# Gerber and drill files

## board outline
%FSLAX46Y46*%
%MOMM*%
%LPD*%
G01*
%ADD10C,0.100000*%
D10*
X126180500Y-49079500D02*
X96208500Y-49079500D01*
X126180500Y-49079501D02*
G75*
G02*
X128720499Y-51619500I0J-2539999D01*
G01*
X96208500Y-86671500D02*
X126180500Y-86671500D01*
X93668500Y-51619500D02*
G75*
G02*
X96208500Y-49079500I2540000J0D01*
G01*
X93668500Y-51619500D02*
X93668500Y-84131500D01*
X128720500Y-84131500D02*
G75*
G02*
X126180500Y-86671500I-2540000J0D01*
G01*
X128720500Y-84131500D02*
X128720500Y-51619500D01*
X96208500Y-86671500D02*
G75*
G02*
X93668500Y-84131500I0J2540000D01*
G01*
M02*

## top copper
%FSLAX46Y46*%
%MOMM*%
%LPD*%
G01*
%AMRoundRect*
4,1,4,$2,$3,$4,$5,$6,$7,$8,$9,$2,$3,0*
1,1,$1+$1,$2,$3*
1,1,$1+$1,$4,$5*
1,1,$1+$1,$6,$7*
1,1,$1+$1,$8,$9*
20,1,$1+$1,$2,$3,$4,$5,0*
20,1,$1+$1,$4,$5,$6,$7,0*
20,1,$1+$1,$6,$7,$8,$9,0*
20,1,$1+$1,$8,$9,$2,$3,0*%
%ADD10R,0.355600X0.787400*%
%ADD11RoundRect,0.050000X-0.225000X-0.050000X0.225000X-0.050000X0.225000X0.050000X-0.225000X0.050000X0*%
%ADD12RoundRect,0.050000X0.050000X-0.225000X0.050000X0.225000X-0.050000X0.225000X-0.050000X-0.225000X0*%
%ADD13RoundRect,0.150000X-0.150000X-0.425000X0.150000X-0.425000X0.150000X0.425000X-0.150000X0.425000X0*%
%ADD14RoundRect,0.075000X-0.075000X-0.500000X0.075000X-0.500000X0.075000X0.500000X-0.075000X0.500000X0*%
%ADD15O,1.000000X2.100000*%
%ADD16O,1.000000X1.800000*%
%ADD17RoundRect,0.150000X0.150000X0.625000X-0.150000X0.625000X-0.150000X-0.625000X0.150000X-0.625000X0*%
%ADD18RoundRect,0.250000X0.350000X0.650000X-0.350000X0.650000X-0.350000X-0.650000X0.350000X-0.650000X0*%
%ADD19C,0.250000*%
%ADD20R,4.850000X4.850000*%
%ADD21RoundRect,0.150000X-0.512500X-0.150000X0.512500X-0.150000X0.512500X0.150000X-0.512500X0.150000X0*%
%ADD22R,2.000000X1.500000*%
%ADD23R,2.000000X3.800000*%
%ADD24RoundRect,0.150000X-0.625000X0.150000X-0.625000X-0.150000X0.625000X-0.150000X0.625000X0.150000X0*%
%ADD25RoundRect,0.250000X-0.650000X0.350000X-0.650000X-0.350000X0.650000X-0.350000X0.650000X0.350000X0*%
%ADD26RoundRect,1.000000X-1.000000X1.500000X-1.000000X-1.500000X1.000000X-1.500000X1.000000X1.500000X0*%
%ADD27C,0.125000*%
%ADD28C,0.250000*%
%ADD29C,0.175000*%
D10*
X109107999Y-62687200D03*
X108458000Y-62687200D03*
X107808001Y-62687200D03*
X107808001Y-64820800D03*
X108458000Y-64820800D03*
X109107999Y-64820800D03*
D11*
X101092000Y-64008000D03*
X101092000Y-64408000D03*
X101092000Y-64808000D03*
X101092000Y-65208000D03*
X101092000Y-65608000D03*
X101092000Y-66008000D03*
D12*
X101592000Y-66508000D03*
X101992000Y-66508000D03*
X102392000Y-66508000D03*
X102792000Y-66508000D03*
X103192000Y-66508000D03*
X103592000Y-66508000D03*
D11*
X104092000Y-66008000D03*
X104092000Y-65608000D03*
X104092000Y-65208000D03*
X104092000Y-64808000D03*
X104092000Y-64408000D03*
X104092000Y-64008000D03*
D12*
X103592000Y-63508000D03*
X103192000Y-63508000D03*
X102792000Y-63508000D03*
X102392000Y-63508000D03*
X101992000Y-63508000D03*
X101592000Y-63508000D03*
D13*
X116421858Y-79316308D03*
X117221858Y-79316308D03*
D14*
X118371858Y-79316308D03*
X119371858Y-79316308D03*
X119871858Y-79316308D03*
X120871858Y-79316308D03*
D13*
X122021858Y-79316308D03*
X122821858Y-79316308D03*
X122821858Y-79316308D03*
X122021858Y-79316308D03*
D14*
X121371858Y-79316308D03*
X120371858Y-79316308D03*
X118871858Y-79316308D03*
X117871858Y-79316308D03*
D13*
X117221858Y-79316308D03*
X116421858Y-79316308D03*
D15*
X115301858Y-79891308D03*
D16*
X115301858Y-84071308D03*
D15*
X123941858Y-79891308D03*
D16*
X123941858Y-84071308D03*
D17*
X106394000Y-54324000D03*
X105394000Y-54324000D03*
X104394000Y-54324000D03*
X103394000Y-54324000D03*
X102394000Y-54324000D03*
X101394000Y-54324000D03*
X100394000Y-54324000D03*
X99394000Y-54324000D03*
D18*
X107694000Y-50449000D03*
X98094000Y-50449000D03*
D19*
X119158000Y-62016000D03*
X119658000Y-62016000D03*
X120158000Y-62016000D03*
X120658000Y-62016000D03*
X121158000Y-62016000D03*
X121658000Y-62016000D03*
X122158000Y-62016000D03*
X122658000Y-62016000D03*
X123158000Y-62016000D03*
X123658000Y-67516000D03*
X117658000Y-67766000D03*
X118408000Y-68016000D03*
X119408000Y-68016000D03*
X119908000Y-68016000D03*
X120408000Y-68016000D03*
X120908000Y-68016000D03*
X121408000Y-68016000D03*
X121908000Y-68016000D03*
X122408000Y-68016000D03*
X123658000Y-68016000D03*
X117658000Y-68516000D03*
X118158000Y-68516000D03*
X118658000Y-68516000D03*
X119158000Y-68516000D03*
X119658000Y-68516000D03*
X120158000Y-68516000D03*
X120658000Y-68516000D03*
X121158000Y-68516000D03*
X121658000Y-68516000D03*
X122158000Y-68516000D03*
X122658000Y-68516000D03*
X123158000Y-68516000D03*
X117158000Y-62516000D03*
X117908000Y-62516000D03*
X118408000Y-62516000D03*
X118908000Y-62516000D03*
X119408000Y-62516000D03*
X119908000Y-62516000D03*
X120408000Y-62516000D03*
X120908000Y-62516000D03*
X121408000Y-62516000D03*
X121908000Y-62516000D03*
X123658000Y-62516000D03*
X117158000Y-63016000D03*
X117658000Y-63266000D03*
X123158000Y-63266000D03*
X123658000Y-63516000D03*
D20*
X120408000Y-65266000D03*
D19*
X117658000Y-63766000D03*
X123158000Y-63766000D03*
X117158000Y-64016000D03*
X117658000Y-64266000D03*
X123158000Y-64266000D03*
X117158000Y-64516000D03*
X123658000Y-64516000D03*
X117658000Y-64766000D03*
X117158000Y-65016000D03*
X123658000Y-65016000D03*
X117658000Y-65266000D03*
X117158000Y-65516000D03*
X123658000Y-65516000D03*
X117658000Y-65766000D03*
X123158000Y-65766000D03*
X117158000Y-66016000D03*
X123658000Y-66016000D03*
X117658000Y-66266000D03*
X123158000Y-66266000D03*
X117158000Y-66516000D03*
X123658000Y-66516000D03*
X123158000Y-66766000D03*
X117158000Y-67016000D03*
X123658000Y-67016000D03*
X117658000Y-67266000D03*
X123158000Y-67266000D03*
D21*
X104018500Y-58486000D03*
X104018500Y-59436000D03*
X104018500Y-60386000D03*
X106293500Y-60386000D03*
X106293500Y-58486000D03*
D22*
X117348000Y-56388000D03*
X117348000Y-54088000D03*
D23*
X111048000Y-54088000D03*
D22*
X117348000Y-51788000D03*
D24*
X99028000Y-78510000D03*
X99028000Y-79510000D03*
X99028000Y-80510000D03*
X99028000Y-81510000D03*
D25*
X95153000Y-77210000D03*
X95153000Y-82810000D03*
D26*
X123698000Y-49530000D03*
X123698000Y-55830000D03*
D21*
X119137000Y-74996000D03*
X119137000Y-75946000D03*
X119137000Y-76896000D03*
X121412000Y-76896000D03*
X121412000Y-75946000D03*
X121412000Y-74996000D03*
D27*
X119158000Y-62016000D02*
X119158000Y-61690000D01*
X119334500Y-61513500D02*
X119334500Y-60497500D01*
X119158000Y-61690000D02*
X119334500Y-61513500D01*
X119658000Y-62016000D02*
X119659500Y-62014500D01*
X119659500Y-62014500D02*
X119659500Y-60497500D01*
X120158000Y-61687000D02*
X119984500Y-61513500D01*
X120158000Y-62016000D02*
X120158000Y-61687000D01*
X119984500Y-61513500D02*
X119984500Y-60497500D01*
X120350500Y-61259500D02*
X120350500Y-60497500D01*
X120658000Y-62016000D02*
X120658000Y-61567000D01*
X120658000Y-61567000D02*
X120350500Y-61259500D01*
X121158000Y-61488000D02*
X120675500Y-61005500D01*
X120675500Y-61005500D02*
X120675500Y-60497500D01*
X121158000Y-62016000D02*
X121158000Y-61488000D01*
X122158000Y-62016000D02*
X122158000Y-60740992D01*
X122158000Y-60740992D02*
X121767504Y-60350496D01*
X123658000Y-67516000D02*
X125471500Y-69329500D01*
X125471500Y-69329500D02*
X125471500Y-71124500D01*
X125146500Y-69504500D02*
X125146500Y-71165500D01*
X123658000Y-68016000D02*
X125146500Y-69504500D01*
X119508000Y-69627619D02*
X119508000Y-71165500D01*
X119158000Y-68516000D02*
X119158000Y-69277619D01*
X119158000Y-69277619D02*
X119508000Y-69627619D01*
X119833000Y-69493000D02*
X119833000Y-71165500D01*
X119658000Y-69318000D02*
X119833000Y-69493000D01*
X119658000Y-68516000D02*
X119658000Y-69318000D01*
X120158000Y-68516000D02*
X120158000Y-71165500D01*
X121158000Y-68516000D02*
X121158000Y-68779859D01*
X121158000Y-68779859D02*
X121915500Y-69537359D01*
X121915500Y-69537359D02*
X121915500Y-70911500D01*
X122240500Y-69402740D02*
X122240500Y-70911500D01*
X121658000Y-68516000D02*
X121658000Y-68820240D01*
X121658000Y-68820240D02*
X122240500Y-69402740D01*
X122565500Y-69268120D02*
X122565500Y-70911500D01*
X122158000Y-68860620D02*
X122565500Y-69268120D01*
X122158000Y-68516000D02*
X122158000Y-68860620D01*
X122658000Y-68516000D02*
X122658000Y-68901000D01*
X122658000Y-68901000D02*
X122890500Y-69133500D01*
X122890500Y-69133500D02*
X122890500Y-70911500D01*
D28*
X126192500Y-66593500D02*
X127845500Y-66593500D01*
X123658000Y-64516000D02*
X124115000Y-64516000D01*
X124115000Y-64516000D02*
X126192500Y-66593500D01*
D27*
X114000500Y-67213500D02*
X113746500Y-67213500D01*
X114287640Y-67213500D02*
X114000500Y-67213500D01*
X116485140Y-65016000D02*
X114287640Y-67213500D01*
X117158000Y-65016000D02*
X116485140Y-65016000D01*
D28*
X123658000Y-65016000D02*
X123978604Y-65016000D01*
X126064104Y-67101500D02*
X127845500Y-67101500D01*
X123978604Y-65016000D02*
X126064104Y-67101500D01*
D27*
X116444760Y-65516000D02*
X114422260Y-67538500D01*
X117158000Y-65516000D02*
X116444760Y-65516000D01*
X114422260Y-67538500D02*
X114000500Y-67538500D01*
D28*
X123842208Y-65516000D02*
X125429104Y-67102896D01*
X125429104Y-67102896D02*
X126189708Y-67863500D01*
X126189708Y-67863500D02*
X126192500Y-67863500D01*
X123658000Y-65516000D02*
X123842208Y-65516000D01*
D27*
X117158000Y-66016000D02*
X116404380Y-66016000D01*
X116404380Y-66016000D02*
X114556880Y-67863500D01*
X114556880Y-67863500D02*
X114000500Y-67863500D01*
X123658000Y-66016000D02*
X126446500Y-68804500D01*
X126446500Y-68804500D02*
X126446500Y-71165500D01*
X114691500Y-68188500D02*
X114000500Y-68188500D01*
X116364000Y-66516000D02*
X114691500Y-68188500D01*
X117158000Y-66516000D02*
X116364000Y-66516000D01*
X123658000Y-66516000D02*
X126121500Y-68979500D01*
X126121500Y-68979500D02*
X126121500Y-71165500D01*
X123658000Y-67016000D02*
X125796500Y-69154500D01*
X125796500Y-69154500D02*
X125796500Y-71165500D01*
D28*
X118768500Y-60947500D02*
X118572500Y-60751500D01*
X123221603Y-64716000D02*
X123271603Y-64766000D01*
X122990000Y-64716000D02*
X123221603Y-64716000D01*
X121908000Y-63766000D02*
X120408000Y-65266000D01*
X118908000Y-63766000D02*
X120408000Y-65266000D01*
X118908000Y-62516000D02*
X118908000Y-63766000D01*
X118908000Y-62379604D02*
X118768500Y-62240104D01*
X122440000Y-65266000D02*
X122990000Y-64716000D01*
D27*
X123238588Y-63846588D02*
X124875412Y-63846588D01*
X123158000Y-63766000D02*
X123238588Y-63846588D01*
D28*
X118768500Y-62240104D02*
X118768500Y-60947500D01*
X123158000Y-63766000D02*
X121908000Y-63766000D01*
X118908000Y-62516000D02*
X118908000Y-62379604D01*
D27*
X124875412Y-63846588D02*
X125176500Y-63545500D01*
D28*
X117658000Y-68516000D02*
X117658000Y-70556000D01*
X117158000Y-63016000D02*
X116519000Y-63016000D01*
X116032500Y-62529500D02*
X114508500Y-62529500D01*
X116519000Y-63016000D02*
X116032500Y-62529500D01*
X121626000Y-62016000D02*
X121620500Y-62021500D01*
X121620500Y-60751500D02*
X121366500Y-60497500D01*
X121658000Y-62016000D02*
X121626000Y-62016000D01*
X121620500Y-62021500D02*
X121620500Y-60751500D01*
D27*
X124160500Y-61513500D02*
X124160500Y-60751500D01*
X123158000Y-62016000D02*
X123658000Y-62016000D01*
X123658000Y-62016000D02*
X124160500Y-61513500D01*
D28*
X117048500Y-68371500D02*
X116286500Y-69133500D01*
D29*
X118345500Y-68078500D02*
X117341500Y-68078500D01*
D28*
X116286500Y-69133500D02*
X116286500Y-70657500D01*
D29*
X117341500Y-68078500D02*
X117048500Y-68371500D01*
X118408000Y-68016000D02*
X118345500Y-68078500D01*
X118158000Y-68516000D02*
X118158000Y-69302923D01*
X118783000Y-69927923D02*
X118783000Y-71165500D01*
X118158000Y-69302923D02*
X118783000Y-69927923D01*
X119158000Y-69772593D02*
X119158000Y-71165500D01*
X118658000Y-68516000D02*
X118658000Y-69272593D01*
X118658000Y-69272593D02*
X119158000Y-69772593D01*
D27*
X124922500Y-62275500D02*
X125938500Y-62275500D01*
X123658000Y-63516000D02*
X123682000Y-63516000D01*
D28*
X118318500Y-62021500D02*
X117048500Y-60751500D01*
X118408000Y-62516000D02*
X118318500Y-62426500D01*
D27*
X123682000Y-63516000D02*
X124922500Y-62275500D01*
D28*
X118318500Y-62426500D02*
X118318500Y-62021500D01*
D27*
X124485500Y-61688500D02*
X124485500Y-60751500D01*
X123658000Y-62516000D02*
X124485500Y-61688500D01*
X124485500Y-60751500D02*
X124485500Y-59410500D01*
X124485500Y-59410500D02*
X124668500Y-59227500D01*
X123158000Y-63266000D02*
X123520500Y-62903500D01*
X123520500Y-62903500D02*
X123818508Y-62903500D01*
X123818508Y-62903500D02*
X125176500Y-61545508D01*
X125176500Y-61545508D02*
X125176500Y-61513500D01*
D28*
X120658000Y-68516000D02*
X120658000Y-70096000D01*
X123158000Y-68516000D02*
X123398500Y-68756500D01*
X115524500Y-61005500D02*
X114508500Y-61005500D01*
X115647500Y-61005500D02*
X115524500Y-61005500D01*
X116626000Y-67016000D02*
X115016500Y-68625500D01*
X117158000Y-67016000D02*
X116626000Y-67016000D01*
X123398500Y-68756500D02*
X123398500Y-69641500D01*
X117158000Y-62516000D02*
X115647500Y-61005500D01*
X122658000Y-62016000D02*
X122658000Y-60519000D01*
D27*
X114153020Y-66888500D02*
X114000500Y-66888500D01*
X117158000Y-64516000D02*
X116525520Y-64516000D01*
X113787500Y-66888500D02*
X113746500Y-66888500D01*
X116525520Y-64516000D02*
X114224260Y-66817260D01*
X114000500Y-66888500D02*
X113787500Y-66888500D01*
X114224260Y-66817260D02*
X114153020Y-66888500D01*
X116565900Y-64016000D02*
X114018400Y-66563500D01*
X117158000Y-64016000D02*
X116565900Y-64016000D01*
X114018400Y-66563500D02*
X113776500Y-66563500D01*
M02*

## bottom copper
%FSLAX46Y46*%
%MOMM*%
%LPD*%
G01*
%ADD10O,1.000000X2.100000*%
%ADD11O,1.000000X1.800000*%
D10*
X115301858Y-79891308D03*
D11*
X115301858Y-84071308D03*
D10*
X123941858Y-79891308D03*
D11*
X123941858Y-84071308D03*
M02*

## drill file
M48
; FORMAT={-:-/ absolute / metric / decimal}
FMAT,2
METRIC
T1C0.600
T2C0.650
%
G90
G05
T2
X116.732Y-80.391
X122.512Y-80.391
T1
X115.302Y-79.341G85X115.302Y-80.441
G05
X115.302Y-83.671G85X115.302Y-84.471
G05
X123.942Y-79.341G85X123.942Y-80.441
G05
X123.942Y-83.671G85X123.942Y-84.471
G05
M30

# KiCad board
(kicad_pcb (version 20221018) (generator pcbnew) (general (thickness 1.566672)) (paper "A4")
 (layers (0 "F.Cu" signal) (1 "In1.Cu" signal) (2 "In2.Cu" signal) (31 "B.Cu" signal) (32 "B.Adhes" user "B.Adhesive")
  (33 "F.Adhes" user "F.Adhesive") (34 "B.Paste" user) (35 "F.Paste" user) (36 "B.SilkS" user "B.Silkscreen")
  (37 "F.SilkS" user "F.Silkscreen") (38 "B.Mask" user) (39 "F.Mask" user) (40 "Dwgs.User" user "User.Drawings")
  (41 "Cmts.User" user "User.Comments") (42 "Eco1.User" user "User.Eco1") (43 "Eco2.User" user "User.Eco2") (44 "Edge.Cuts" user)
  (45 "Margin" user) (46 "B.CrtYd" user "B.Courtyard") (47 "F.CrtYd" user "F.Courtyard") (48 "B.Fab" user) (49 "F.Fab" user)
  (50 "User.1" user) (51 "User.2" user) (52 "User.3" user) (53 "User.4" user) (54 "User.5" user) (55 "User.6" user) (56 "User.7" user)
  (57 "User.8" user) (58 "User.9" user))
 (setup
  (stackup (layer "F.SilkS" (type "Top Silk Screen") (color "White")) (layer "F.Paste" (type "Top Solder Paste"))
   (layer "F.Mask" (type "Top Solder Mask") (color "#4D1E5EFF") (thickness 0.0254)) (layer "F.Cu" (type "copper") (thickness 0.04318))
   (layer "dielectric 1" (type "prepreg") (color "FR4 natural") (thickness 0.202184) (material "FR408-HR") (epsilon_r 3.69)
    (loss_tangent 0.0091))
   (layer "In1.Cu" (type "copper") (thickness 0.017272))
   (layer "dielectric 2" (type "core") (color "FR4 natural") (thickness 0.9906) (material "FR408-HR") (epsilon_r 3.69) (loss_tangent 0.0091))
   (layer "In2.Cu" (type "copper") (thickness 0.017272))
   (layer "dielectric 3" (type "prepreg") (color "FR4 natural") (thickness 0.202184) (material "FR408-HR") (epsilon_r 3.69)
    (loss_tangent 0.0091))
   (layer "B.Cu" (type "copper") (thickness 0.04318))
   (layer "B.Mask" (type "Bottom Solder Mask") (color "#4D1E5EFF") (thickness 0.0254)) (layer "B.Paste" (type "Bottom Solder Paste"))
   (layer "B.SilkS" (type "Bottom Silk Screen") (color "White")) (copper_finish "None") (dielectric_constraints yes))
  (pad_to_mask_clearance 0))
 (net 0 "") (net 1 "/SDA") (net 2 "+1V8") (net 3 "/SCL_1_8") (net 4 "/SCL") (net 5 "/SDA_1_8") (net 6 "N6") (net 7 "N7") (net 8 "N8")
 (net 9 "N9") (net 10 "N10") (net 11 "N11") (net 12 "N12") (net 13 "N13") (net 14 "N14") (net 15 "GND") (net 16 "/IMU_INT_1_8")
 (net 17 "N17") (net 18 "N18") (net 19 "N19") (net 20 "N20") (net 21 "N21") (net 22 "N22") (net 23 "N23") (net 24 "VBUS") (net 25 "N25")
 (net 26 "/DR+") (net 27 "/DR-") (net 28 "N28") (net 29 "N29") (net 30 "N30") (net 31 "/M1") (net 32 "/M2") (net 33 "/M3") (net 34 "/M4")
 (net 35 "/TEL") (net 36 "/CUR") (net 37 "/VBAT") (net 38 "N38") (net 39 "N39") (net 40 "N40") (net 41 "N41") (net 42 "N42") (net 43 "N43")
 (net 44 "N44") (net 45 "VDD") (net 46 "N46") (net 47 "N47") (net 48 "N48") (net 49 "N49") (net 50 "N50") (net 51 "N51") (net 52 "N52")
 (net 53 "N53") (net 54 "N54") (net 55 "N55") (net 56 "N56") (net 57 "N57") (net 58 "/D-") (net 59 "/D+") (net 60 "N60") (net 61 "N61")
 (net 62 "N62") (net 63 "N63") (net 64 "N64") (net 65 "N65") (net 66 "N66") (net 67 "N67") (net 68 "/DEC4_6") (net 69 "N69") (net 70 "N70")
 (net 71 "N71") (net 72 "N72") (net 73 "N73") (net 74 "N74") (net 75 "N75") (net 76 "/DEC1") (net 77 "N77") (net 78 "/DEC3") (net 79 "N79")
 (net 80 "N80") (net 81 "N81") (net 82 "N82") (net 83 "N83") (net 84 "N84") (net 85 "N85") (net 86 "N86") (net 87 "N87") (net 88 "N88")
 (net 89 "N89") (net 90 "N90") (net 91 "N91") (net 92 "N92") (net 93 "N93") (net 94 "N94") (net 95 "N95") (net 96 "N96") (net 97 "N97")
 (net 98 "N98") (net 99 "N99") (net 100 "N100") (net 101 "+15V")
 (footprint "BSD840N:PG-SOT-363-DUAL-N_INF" (layer "F.Cu") (at 108.458 63.754 -90)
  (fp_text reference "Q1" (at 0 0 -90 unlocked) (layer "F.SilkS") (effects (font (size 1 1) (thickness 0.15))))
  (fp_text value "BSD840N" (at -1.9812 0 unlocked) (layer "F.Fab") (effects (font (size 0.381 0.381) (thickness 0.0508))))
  (pad "1" smd rect (at -1.0668 -0.649999 270) (size 0.7874 0.3556) (layers "F.Cu" "F.Paste" "F.Mask") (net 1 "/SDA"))
  (pad "2" smd rect (at -1.0668 0 270) (size 0.7874 0.3556) (layers "F.Cu" "F.Paste" "F.Mask") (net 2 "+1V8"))
  (pad "3" smd rect (at -1.0668 0.649999 270) (size 0.7874 0.3556) (layers "F.Cu" "F.Paste" "F.Mask") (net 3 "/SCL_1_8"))
  (pad "4" smd rect (at 1.0668 0.649999 270) (size 0.7874 0.3556) (layers "F.Cu" "F.Paste" "F.Mask") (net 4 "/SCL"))
  (pad "5" smd rect (at 1.0668 0 270) (size 0.7874 0.3556) (layers "F.Cu" "F.Paste" "F.Mask") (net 2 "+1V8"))
  (pad "6" smd rect (at 1.0668 -0.649999 270) (size 0.7874 0.3556) (layers "F.Cu" "F.Paste" "F.Mask") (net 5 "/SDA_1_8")))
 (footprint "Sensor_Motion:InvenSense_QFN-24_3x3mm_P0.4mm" (layer "F.Cu") (at 102.592 65.008)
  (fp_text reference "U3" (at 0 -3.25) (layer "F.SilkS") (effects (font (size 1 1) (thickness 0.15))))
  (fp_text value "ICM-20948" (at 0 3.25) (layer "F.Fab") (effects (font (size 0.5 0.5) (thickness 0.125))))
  (pad "1" smd roundrect (at -1.5 -1) (size 0.55 0.2) (layers "F.Cu" "F.Paste" "F.Mask") (roundrect_rratio 0.25) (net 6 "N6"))
  (pad "2" smd roundrect (at -1.5 -0.6) (size 0.55 0.2) (layers "F.Cu" "F.Paste" "F.Mask") (roundrect_rratio 0.25) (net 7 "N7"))
  (pad "3" smd roundrect (at -1.5 -0.2) (size 0.55 0.2) (layers "F.Cu" "F.Paste" "F.Mask") (roundrect_rratio 0.25) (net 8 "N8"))
  (pad "4" smd roundrect (at -1.5 0.2) (size 0.55 0.2) (layers "F.Cu" "F.Paste" "F.Mask") (roundrect_rratio 0.25) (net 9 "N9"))
  (pad "5" smd roundrect (at -1.5 0.6) (size 0.55 0.2) (layers "F.Cu" "F.Paste" "F.Mask") (roundrect_rratio 0.25) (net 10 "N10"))
  (pad "6" smd roundrect (at -1.5 1) (size 0.55 0.2) (layers "F.Cu" "F.Paste" "F.Mask") (roundrect_rratio 0.25) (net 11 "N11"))
  (pad "7" smd roundrect (at -1 1.5 90) (size 0.55 0.2) (layers "F.Cu" "F.Paste" "F.Mask") (roundrect_rratio 0.25) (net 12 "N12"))
  (pad "8" smd roundrect (at -0.6 1.5 90) (size 0.55 0.2) (layers "F.Cu" "F.Paste" "F.Mask") (roundrect_rratio 0.25) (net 2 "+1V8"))
  (pad "9" smd roundrect (at -0.2 1.5 90) (size 0.55 0.2) (layers "F.Cu" "F.Paste" "F.Mask") (roundrect_rratio 0.25) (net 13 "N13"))
  (pad "10" smd roundrect (at 0.2 1.5 90) (size 0.55 0.2) (layers "F.Cu" "F.Paste" "F.Mask") (roundrect_rratio 0.25) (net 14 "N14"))
  (pad "11" smd roundrect (at 0.6 1.5 90) (size 0.55 0.2) (layers "F.Cu" "F.Paste" "F.Mask") (roundrect_rratio 0.25) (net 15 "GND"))
  (pad "12" smd roundrect (at 1 1.5 90) (size 0.55 0.2) (layers "F.Cu" "F.Paste" "F.Mask") (roundrect_rratio 0.25) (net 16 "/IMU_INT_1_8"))
  (pad "13" smd roundrect (at 1.5 1) (size 0.55 0.2) (layers "F.Cu" "F.Paste" "F.Mask") (roundrect_rratio 0.25) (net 2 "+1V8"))
  (pad "14" smd roundrect (at 1.5 0.6) (size 0.55 0.2) (layers "F.Cu" "F.Paste" "F.Mask") (roundrect_rratio 0.25) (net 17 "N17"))
  (pad "15" smd roundrect (at 1.5 0.2) (size 0.55 0.2) (layers "F.Cu" "F.Paste" "F.Mask") (roundrect_rratio 0.25) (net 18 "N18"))
  (pad "16" smd roundrect (at 1.5 -0.2) (size 0.55 0.2) (layers "F.Cu" "F.Paste" "F.Mask") (roundrect_rratio 0.25) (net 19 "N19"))
  (pad "17" smd roundrect (at 1.5 -0.6) (size 0.55 0.2) (layers "F.Cu" "F.Paste" "F.Mask") (roundrect_rratio 0.25) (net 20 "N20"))
  (pad "18" smd roundrect (at 1.5 -1) (size 0.55 0.2) (layers "F.Cu" "F.Paste" "F.Mask") (roundrect_rratio 0.25) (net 15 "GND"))
  (pad "19" smd roundrect (at 1 -1.5 90) (size 0.55 0.2) (layers "F.Cu" "F.Paste" "F.Mask") (roundrect_rratio 0.25) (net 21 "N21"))
  (pad "20" smd roundrect (at 0.6 -1.5 90) (size 0.55 0.2) (layers "F.Cu" "F.Paste" "F.Mask") (roundrect_rratio 0.25) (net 15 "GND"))
  (pad "21" smd roundrect (at 0.2 -1.5 90) (size 0.55 0.2) (layers "F.Cu" "F.Paste" "F.Mask") (roundrect_rratio 0.25) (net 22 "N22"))
  (pad "22" smd roundrect (at -0.2 -1.5 90) (size 0.55 0.2) (layers "F.Cu" "F.Paste" "F.Mask") (roundrect_rratio 0.25) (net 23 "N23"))
  (pad "23" smd roundrect (at -0.6 -1.5 90) (size 0.55 0.2) (layers "F.Cu" "F.Paste" "F.Mask") (roundrect_rratio 0.25) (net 3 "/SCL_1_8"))
  (pad "24" smd roundrect (at -1 -1.5 90) (size 0.55 0.2) (layers "F.Cu" "F.Paste" "F.Mask") (roundrect_rratio 0.25) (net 5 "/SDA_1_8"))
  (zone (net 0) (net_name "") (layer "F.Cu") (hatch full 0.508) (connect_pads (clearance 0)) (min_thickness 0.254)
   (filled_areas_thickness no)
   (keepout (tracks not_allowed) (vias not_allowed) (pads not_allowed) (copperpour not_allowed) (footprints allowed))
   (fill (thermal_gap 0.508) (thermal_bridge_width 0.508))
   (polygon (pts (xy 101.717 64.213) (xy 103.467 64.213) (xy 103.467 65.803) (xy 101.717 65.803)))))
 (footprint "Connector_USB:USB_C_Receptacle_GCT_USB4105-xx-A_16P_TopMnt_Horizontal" (layer "F.Cu") (at 119.621858 82.996308)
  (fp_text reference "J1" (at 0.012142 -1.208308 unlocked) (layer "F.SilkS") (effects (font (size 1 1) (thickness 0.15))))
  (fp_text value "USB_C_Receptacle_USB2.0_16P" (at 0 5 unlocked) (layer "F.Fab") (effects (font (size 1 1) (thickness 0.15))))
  (pad "" np_thru_hole circle (at -2.89 -2.605) (size 0.65 0.65) (drill 0.65) (layers "F&B.Cu" "*.Mask"))
  (pad "" np_thru_hole circle (at 2.89 -2.605) (size 0.65 0.65) (drill 0.65) (layers "F&B.Cu" "*.Mask"))
  (pad "A1" smd roundrect (at -3.2 -3.68) (size 0.6 1.15) (layers "F.Cu" "F.Paste" "F.Mask") (roundrect_rratio 0.25) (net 15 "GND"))
  (pad "A4" smd roundrect (at -2.4 -3.68) (size 0.6 1.15) (layers "F.Cu" "F.Paste" "F.Mask") (roundrect_rratio 0.25) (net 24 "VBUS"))
  (pad "A5" smd roundrect (at -1.25 -3.68) (size 0.3 1.15) (layers "F.Cu" "F.Paste" "F.Mask") (roundrect_rratio 0.25) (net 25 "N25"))
  (pad "A6" smd roundrect (at -0.25 -3.68) (size 0.3 1.15) (layers "F.Cu" "F.Paste" "F.Mask") (roundrect_rratio 0.25) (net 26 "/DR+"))
  (pad "A7" smd roundrect (at 0.25 -3.68) (size 0.3 1.15) (layers "F.Cu" "F.Paste" "F.Mask") (roundrect_rratio 0.25) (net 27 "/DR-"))
  (pad "A8" smd roundrect (at 1.25 -3.68) (size 0.3 1.15) (layers "F.Cu" "F.Paste" "F.Mask") (roundrect_rratio 0.25) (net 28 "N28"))
  (pad "A9" smd roundrect (at 2.4 -3.68) (size 0.6 1.15) (layers "F.Cu" "F.Paste" "F.Mask") (roundrect_rratio 0.25) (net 24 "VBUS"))
  (pad "A12" smd roundrect (at 3.2 -3.68) (size 0.6 1.15) (layers "F.Cu" "F.Paste" "F.Mask") (roundrect_rratio 0.25) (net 15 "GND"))
  (pad "B1" smd roundrect (at 3.2 -3.68) (size 0.6 1.15) (layers "F.Cu" "F.Paste" "F.Mask") (roundrect_rratio 0.25) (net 15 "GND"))
  (pad "B4" smd roundrect (at 2.4 -3.68) (size 0.6 1.15) (layers "F.Cu" "F.Paste" "F.Mask") (roundrect_rratio 0.25) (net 24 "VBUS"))
  (pad "B5" smd roundrect (at 1.75 -3.68) (size 0.3 1.15) (layers "F.Cu" "F.Paste" "F.Mask") (roundrect_rratio 0.25) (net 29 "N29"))
  (pad "B6" smd roundrect (at 0.75 -3.68) (size 0.3 1.15) (layers "F.Cu" "F.Paste" "F.Mask") (roundrect_rratio 0.25) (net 26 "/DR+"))
  (pad "B7" smd roundrect (at -0.75 -3.68) (size 0.3 1.15) (layers "F.Cu" "F.Paste" "F.Mask") (roundrect_rratio 0.25) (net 27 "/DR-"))
  (pad "B8" smd roundrect (at -1.75 -3.68) (size 0.3 1.15) (layers "F.Cu" "F.Paste" "F.Mask") (roundrect_rratio 0.25) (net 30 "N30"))
  (pad "B9" smd roundrect (at -2.4 -3.68) (size 0.6 1.15) (layers "F.Cu" "F.Paste" "F.Mask") (roundrect_rratio 0.25) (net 24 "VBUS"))
  (pad "B12" smd roundrect (at -3.2 -3.68) (size 0.6 1.15) (layers "F.Cu" "F.Paste" "F.Mask") (roundrect_rratio 0.25) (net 15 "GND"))
  (pad "S1" thru_hole oval (at -4.32 -3.105) (size 1 2.1) (drill oval 0.6 1.7) (layers "*.Cu" "*.Mask" "F.Paste") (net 15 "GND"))
  (pad "S1" thru_hole oval (at -4.32 1.075) (size 1 1.8) (drill oval 0.6 1.4) (layers "*.Cu" "*.Mask" "F.Paste") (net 15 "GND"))
  (pad "S1" thru_hole oval (at 4.32 -3.105) (size 1 2.1) (drill oval 0.6 1.7) (layers "*.Cu" "*.Mask" "F.Paste") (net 15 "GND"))
  (pad "S1" thru_hole oval (at 4.32 1.075) (size 1 1.8) (drill oval 0.6 1.4) (layers "*.Cu" "*.Mask" "F.Paste") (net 15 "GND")))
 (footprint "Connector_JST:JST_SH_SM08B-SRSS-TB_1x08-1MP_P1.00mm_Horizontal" (layer "F.Cu") (at 102.894 52.324 180)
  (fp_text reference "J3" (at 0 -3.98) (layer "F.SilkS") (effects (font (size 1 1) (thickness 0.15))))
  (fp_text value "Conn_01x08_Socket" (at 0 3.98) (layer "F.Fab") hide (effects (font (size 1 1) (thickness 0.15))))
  (pad "1" smd roundrect (at -3.5 -2 180) (size 0.6 1.55) (layers "F.Cu" "F.Paste" "F.Mask") (roundrect_rratio 0.25) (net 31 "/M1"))
  (pad "2" smd roundrect (at -2.5 -2 180) (size 0.6 1.55) (layers "F.Cu" "F.Paste" "F.Mask") (roundrect_rratio 0.25) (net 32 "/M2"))
  (pad "3" smd roundrect (at -1.5 -2 180) (size 0.6 1.55) (layers "F.Cu" "F.Paste" "F.Mask") (roundrect_rratio 0.25) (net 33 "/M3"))
  (pad "4" smd roundrect (at -0.5 -2 180) (size 0.6 1.55) (layers "F.Cu" "F.Paste" "F.Mask") (roundrect_rratio 0.25) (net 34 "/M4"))
  (pad "5" smd roundrect (at 0.5 -2 180) (size 0.6 1.55) (layers "F.Cu" "F.Paste" "F.Mask") (roundrect_rratio 0.25) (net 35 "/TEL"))
  (pad "6" smd roundrect (at 1.5 -2 180) (size 0.6 1.55) (layers "F.Cu" "F.Paste" "F.Mask") (roundrect_rratio 0.25) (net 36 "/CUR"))
  (pad "7" smd roundrect (at 2.5 -2 180) (size 0.6 1.55) (layers "F.Cu" "F.Paste" "F.Mask") (roundrect_rratio 0.25) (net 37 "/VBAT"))
  (pad "8" smd roundrect (at 3.5 -2 180) (size 0.6 1.55) (layers "F.Cu" "F.Paste" "F.Mask") (roundrect_rratio 0.25) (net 15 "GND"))
  (pad "MP" smd roundrect (at -4.8 1.875 180) (size 1.2 1.8) (layers "F.Cu" "F.Paste" "F.Mask") (roundrect_rratio 0.208333))
  (pad "MP" smd roundrect (at 4.8 1.875 180) (size 1.2 1.8) (layers "F.Cu" "F.Paste" "F.Mask") (roundrect_rratio 0.208333)))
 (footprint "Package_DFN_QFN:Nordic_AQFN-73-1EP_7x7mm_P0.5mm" (layer "F.Cu") (at 120.408 65.266)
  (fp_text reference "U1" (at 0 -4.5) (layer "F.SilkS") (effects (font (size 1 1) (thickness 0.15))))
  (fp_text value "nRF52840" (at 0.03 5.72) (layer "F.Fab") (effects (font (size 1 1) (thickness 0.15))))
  (pad "" smd rect (at -1.2125 -1.2125 180) (size 2 2) (layers "F.Paste"))
  (pad "" smd rect (at -1.2125 1.2125 180) (size 2 2) (layers "F.Paste"))
  (pad "" smd rect (at 1.2125 -1.2125 180) (size 2 2) (layers "F.Paste"))
  (pad "" smd rect (at 1.2125 1.2125 180) (size 2 2) (layers "F.Paste"))
  (pad "A8" smd circle (at -1.25 -3.25 180) (size 0.25 0.25) (layers "F.Cu" "F.Paste" "F.Mask") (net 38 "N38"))
  (pad "A10" smd circle (at -0.75 -3.25 180) (size 0.25 0.25) (layers "F.Cu" "F.Paste" "F.Mask") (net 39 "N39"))
  (pad "A12" smd circle (at -0.25 -3.25 180) (size 0.25 0.25) (layers "F.Cu" "F.Paste" "F.Mask") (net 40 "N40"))
  (pad "A14" smd circle (at 0.25 -3.25 180) (size 0.25 0.25) (layers "F.Cu" "F.Paste" "F.Mask") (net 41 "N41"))
  (pad "A16" smd circle (at 0.75 -3.25 180) (size 0.25 0.25) (layers "F.Cu" "F.Paste" "F.Mask") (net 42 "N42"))
  (pad "A18" smd circle (at 1.25 -3.25 180) (size 0.25 0.25) (layers "F.Cu" "F.Paste" "F.Mask") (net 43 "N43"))
  (pad "A20" smd circle (at 1.75 -3.25 180) (size 0.25 0.25) (layers "F.Cu" "F.Paste" "F.Mask") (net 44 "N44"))
  (pad "A22" smd circle (at 2.25 -3.25 180) (size 0.25 0.25) (layers "F.Cu" "F.Paste" "F.Mask") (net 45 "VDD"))
  (pad "A23" smd circle (at 2.75 -3.25 180) (size 0.25 0.25) (layers "F.Cu" "F.Paste" "F.Mask") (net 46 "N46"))
  (pad "AA24" smd circle (at 3.25 2.25 180) (size 0.25 0.25) (layers "F.Cu" "F.Paste" "F.Mask") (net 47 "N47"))
  (pad "AB2" smd circle (at -2.75 2.5 180) (size 0.25 0.25) (layers "F.Cu" "F.Paste" "F.Mask") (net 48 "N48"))
  (pad "AC5" smd circle (at -2 2.75 180) (size 0.25 0.25) (layers "F.Cu" "F.Paste" "F.Mask") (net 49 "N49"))
  (pad "AC9" smd circle (at -1 2.75 180) (size 0.25 0.25) (layers "F.Cu" "F.Paste" "F.Mask") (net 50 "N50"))
  (pad "AC11" smd circle (at -0.5 2.75 180) (size 0.25 0.25) (layers "F.Cu" "F.Paste" "F.Mask") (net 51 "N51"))
  (pad "AC13" smd circle (at 0 2.75 180) (size 0.25 0.25) (layers "F.Cu" "F.Paste" "F.Mask") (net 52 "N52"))
  (pad "AC15" smd circle (at 0.5 2.75 180) (size 0.25 0.25) (layers "F.Cu" "F.Paste" "F.Mask") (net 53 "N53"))
  (pad "AC17" smd circle (at 1 2.75 180) (size 0.25 0.25) (layers "F.Cu" "F.Paste" "F.Mask") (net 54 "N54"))
  (pad "AC19" smd circle (at 1.5 2.75 180) (size 0.25 0.25) (layers "F.Cu" "F.Paste" "F.Mask") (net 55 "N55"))
  (pad "AC21" smd circle (at 2 2.75 180) (size 0.25 0.25) (layers "F.Cu" "F.Paste" "F.Mask") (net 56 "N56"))
  (pad "AC24" smd circle (at 3.25 2.75 180) (size 0.25 0.25) (layers "F.Cu" "F.Paste" "F.Mask") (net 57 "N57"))
  (pad "AD2" smd circle (at -2.75 3.25 180) (size 0.25 0.25) (layers "F.Cu" "F.Paste" "F.Mask") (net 24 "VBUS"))
  (pad "AD4" smd circle (at -2.25 3.25 180) (size 0.25 0.25) (layers "F.Cu" "F.Paste" "F.Mask") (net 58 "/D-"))
  (pad "AD6" smd circle (at -1.75 3.25 180) (size 0.25 0.25) (layers "F.Cu" "F.Paste" "F.Mask") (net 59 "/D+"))
  (pad "AD8" smd circle (at -1.25 3.25 180) (size 0.25 0.25) (layers "F.Cu" "F.Paste" "F.Mask") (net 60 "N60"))
  (pad "AD10" smd circle (at -0.75 3.25 180) (size 0.25 0.25) (layers "F.Cu" "F.Paste" "F.Mask") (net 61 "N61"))
  (pad "AD12" smd circle (at -0.25 3.25 180) (size 0.25 0.25) (layers "F.Cu" "F.Paste" "F.Mask") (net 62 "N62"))
  (pad "AD14" smd circle (at 0.25 3.25 180) (size 0.25 0.25) (layers "F.Cu" "F.Paste" "F.Mask") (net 45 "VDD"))
  (pad "AD16" smd circle (at 0.75 3.25 180) (size 0.25 0.25) (layers "F.Cu" "F.Paste" "F.Mask") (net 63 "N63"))
  (pad "AD18" smd circle (at 1.25 3.25 180) (size 0.25 0.25) (layers "F.Cu" "F.Paste" "F.Mask") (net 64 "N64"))
  (pad "AD20" smd circle (at 1.75 3.25 180) (size 0.25 0.25) (layers "F.Cu" "F.Paste" "F.Mask") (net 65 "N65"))
  (pad "AD22" smd circle (at 2.25 3.25 180) (size 0.25 0.25) (layers "F.Cu" "F.Paste" "F.Mask") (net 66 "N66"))
  (pad "AD23" smd circle (at 2.75 3.25 180) (size 0.25 0.25) (layers "F.Cu" "F.Paste" "F.Mask") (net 45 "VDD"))
  (pad "B1" smd circle (at -3.25 -2.75 180) (size 0.25 0.25) (layers "F.Cu" "F.Paste" "F.Mask") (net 45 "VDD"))
  (pad "B3" smd circle (at -2.5 -2.75 180) (size 0.25 0.25) (layers "F.Cu" "F.Paste" "F.Mask") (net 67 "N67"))
  (pad "B5" smd circle (at -2 -2.75 180) (size 0.25 0.25) (layers "F.Cu" "F.Paste" "F.Mask") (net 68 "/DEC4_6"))
  (pad "B7" smd circle (at -1.5 -2.75 180) (size 0.25 0.25) (layers "F.Cu" "F.Paste" "F.Mask") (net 15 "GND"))
  (pad "B9" smd circle (at -1 -2.75 180) (size 0.25 0.25) (layers "F.Cu" "F.Paste" "F.Mask") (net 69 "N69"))
  (pad "B11" smd circle (at -0.5 -2.75 180) (size 0.25 0.25) (layers "F.Cu" "F.Paste" "F.Mask") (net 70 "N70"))
  (pad "B13" smd circle (at 0 -2.75 180) (size 0.25 0.25) (layers "F.Cu" "F.Paste" "F.Mask") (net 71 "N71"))
  (pad "B15" smd circle (at 0.5 -2.75 180) (size 0.25 0.25) (layers "F.Cu" "F.Paste" "F.Mask") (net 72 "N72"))
  (pad "B17" smd circle (at 1 -2.75 180) (size 0.25 0.25) (layers "F.Cu" "F.Paste" "F.Mask") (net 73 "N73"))
  (pad "B19" smd circle (at 1.5 -2.75 180) (size 0.25 0.25) (layers "F.Cu" "F.Paste" "F.Mask") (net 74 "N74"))
  (pad "B24" smd circle (at 3.25 -2.75 180) (size 0.25 0.25) (layers "F.Cu" "F.Paste" "F.Mask") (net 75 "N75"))
  (pad "C1" smd circle (at -3.25 -2.25 180) (size 0.25 0.25) (layers "F.Cu" "F.Paste" "F.Mask") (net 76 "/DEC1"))
  (pad "D2" smd circle (at -2.75 -2 180) (size 0.25 0.25) (layers "F.Cu" "F.Paste" "F.Mask") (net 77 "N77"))
  (pad "D23" smd circle (at 2.75 -2 180) (size 0.25 0.25) (layers "F.Cu" "F.Paste" "F.Mask") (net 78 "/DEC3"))
  (pad "E24" smd circle (at 3.25 -1.75 180) (size 0.25 0.25) (layers "F.Cu" "F.Paste" "F.Mask") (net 68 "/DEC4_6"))
  (pad "EP" smd rect (at 0 0 180) (size 4.85 4.85) (layers "F.Cu" "F.Mask"))
  (pad "F2" smd circle (at -2.75 -1.5 180) (size 0.25 0.25) (layers "F.Cu" "F.Paste" "F.Mask") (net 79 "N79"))
  (pad "F23" smd circle (at 2.75 -1.5 180) (size 0.25 0.25) (layers "F.Cu" "F.Paste" "F.Mask") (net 15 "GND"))
  (pad "G1" smd circle (at -3.25 -1.25 180) (size 0.25 0.25) (layers "F.Cu" "F.Paste" "F.Mask") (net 1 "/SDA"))
  (pad "H2" smd circle (at -2.75 -1 180) (size 0.25 0.25) (layers "F.Cu" "F.Paste" "F.Mask") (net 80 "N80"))
  (pad "H23" smd circle (at 2.75 -1 180) (size 0.25 0.25) (layers "F.Cu" "F.Paste" "F.Mask") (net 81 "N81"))
  (pad "J1" smd circle (at -3.25 -0.75 180) (size 0.25 0.25) (layers "F.Cu" "F.Paste" "F.Mask") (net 4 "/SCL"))
  (pad "J24" smd circle (at 3.25 -0.75 180) (size 0.25 0.25) (layers "F.Cu" "F.Paste" "F.Mask") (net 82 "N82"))
  (pad "K2" smd circle (at -2.75 -0.5 180) (size 0.25 0.25) (layers "F.Cu" "F.Paste" "F.Mask") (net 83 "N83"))
  (pad "L1" smd circle (at -3.25 -0.25 180) (size 0.25 0.25) (layers "F.Cu" "F.Paste" "F.Mask") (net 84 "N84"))
  (pad "L24" smd circle (at 3.25 -0.25 180) (size 0.25 0.25) (layers "F.Cu" "F.Paste" "F.Mask") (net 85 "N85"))
  (pad "M2" smd circle (at -2.75 0 180) (size 0.25 0.25) (layers "F.Cu" "F.Paste" "F.Mask") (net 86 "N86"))
  (pad "N1" smd circle (at -3.25 0.25 180) (size 0.25 0.25) (layers "F.Cu" "F.Paste" "F.Mask") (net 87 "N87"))
  (pad "N24" smd circle (at 3.25 0.25 180) (size 0.25 0.25) (layers "F.Cu" "F.Paste" "F.Mask") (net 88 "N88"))
  (pad "P2" smd circle (at -2.75 0.5 180) (size 0.25 0.25) (layers "F.Cu" "F.Paste" "F.Mask") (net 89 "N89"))
  (pad "P23" smd circle (at 2.75 0.5 180) (size 0.25 0.25) (layers "F.Cu" "F.Paste" "F.Mask") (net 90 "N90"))
  (pad "R1" smd circle (at -3.25 0.75 180) (size 0.25 0.25) (layers "F.Cu" "F.Paste" "F.Mask") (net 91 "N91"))
  (pad "R24" smd circle (at 3.25 0.75 180) (size 0.25 0.25) (layers "F.Cu" "F.Paste" "F.Mask") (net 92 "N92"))
  (pad "T2" smd circle (at -2.75 1 180) (size 0.25 0.25) (layers "F.Cu" "F.Paste" "F.Mask") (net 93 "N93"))
  (pad "T23" smd circle (at 2.75 1 180) (size 0.25 0.25) (layers "F.Cu" "F.Paste" "F.Mask") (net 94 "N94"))
  (pad "U1" smd circle (at -3.25 1.25 180) (size 0.25 0.25) (layers "F.Cu" "F.Paste" "F.Mask") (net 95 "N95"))
  (pad "U24" smd circle (at 3.25 1.25 180) (size 0.25 0.25) (layers "F.Cu" "F.Paste" "F.Mask") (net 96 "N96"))
  (pad "V23" smd circle (at 2.75 1.5 180) (size 0.25 0.25) (layers "F.Cu" "F.Paste" "F.Mask") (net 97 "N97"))
  (pad "W1" smd circle (at -3.25 1.75 180) (size 0.25 0.25) (layers "F.Cu" "F.Paste" "F.Mask") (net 45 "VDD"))
  (pad "W24" smd circle (at 3.25 1.75 180) (size 0.25 0.25) (layers "F.Cu" "F.Paste" "F.Mask") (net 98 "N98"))
  (pad "Y2" smd circle (at -2.75 2 180) (size 0.25 0.25) (layers "F.Cu" "F.Paste" "F.Mask") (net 24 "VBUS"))
  (pad "Y23" smd circle (at 2.75 2 180) (size 0.25 0.25) (layers "F.Cu" "F.Paste" "F.Mask") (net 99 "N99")))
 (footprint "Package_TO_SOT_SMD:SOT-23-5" (layer "F.Cu") (at 105.156 59.436)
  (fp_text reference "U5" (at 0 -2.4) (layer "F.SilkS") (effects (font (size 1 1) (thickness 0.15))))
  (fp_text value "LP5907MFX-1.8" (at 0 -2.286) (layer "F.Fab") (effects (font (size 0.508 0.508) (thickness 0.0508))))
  (pad "1" smd roundrect (at -1.1375 -0.95) (size 1.325 0.6) (layers "F.Cu" "F.Paste" "F.Mask") (roundrect_rratio 0.25) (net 45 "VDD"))
  (pad "2" smd roundrect (at -1.1375 0) (size 1.325 0.6) (layers "F.Cu" "F.Paste" "F.Mask") (roundrect_rratio 0.25) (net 15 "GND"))
  (pad "3" smd roundrect (at -1.1375 0.95) (size 1.325 0.6) (layers "F.Cu" "F.Paste" "F.Mask") (roundrect_rratio 0.25) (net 45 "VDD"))
  (pad "4" smd roundrect (at 1.1375 0.95) (size 1.325 0.6) (layers "F.Cu" "F.Paste" "F.Mask") (roundrect_rratio 0.25) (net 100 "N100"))
  (pad "5" smd roundrect (at 1.1375 -0.95) (size 1.325 0.6) (layers "F.Cu" "F.Paste" "F.Mask") (roundrect_rratio 0.25) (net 2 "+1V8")))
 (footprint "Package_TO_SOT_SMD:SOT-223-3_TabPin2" (layer "F.Cu") (at 114.198 54.088 180)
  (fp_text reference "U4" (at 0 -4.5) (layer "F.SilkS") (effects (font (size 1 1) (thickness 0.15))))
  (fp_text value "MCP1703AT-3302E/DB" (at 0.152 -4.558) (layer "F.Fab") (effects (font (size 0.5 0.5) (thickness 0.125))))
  (pad "1" smd rect (at -3.15 -2.3 180) (size 2 1.5) (layers "F.Cu" "F.Paste" "F.Mask") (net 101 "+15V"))
  (pad "2" smd rect (at -3.15 0 180) (size 2 1.5) (layers "F.Cu" "F.Paste" "F.Mask") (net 15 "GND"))
  (pad "2" smd rect (at 3.15 0 180) (size 2 3.8) (layers "F.Cu" "F.Paste" "F.Mask") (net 15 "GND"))
  (pad "3" smd rect (at -3.15 2.3 180) (size 2 1.5) (layers "F.Cu" "F.Paste" "F.Mask") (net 45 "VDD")))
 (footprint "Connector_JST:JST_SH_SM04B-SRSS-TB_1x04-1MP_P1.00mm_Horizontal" (layer "F.Cu") (at 97.028 80.01 -90)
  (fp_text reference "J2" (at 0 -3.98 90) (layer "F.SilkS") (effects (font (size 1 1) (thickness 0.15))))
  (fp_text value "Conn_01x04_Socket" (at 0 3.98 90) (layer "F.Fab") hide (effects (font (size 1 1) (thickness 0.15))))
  (pad "1" smd roundrect (at -1.5 -2 270) (size 0.6 1.55) (layers "F.Cu" "F.Paste" "F.Mask") (roundrect_rratio 0.25) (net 15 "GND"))
  (pad "2" smd roundrect (at -0.5 -2 270) (size 0.6 1.55) (layers "F.Cu" "F.Paste" "F.Mask") (roundrect_rratio 0.25) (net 45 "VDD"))
  (pad "3" smd roundrect (at 0.5 -2 270) (size 0.6 1.55) (layers "F.Cu" "F.Paste" "F.Mask") (roundrect_rratio 0.25) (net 4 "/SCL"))
  (pad "4" smd roundrect (at 1.5 -2 270) (size 0.6 1.55) (layers "F.Cu" "F.Paste" "F.Mask") (roundrect_rratio 0.25) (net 1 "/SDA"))
  (pad "MP" smd roundrect (at -2.8 1.875 270) (size 1.2 1.8) (layers "F.Cu" "F.Paste" "F.Mask") (roundrect_rratio 0.208333))
  (pad "MP" smd roundrect (at 2.8 1.875 270) (size 1.2 1.8) (layers "F.Cu" "F.Paste" "F.Mask") (roundrect_rratio 0.208333)))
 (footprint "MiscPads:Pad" (layer "F.Cu") (at 120.498 52.73 -90)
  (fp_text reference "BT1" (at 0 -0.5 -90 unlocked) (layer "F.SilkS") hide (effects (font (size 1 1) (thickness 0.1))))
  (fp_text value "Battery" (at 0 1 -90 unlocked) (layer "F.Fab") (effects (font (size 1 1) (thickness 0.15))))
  (pad "1" smd roundrect (at -3.2 -3.2 270) (size 5 4) (layers "F.Cu" "F.Paste" "F.Mask") (roundrect_rratio 0.25) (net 101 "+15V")
   (thermal_bridge_angle 45))
  (pad "2" smd roundrect (at 3.1 -3.2 270) (size 5 4) (layers "F.Cu" "F.Paste" "F.Mask") (roundrect_rratio 0.25) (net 15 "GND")
   (thermal_bridge_angle 45)))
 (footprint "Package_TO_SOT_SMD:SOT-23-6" (layer "F.Cu") (at 120.2745 75.946)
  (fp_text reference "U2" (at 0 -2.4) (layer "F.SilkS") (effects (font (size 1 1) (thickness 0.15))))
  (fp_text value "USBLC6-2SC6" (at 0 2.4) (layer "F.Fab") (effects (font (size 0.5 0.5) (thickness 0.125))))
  (pad "1" smd roundrect (at -1.1375 -0.95) (size 1.325 0.6) (layers "F.Cu" "F.Paste" "F.Mask") (roundrect_rratio 0.25) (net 59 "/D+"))
  (pad "2" smd roundrect (at -1.1375 0) (size 1.325 0.6) (layers "F.Cu" "F.Paste" "F.Mask") (roundrect_rratio 0.25) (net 15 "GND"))
  (pad "3" smd roundrect (at -1.1375 0.95) (size 1.325 0.6) (layers "F.Cu" "F.Paste" "F.Mask") (roundrect_rratio 0.25) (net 58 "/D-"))
  (pad "4" smd roundrect (at 1.1375 0.95) (size 1.325 0.6) (layers "F.Cu" "F.Paste" "F.Mask") (roundrect_rratio 0.25) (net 27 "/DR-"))
  (pad "5" smd roundrect (at 1.1375 0) (size 1.325 0.6) (layers "F.Cu" "F.Paste" "F.Mask") (roundrect_rratio 0.25) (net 45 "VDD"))
  (pad "6" smd roundrect (at 1.1375 -0.95) (size 1.325 0.6) (layers "F.Cu" "F.Paste" "F.Mask") (roundrect_rratio 0.25) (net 26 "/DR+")))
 (gr_line (start 126.1805 49.0795) (end 96.2085 49.0795) (stroke (width 0.1) (type default)) (layer "Edge.Cuts"))
 (gr_arc (start 126.1805 49.079501) (mid 127.976551 49.823449) (end 128.720499 51.6195) (stroke (width 0.1) (type default))
  (layer "Edge.Cuts"))
 (gr_line (start 96.2085 86.6715) (end 126.1805 86.6715) (stroke (width 0.1) (type default)) (layer "Edge.Cuts"))
 (gr_arc (start 93.6685 51.6195) (mid 94.412449 49.823449) (end 96.2085 49.0795) (stroke (width 0.1) (type default)) (layer "Edge.Cuts"))
 (gr_line (start 93.6685 51.6195) (end 93.6685 84.1315) (stroke (width 0.1) (type default)) (layer "Edge.Cuts"))
 (gr_arc (start 128.7205 84.1315) (mid 127.976551 85.927551) (end 126.1805 86.6715) (stroke (width 0.1) (type default)) (layer "Edge.Cuts"))
 (gr_line (start 128.7205 84.1315) (end 128.7205 51.6195) (stroke (width 0.1) (type default)) (layer "Edge.Cuts"))
 (gr_arc (start 96.2085 86.6715) (mid 94.412449 85.927551) (end 93.6685 84.1315) (stroke (width 0.1) (type default)) (layer "Edge.Cuts"))
 (segment (start 119.158 62.016) (end 119.158 61.69) (width 0.125) (layer "F.Cu") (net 38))
 (segment (start 119.3345 61.5135) (end 119.3345 60.4975) (width 0.125) (layer "F.Cu") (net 38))
 (segment (start 119.158 61.69) (end 119.3345 61.5135) (width 0.125) (layer "F.Cu") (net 38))
 (segment (start 119.658 62.016) (end 119.6595 62.0145) (width 0.125) (layer "F.Cu") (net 39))
 (segment (start 119.6595 62.0145) (end 119.6595 60.4975) (width 0.125) (layer "F.Cu") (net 39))
 (segment (start 120.158 61.687) (end 119.9845 61.5135) (width 0.125) (layer "F.Cu") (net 40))
 (segment (start 120.158 62.016) (end 120.158 61.687) (width 0.125) (layer "F.Cu") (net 40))
 (segment (start 119.9845 61.5135) (end 119.9845 60.4975) (width 0.125) (layer "F.Cu") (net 40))
 (segment (start 120.3505 61.2595) (end 120.3505 60.4975) (width 0.125) (layer "F.Cu") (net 41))
 (segment (start 120.658 62.016) (end 120.658 61.567) (width 0.125) (layer "F.Cu") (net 41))
 (segment (start 120.658 61.567) (end 120.3505 61.2595) (width 0.125) (layer "F.Cu") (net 41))
 (segment (start 121.158 61.488) (end 120.6755 61.0055) (width 0.125) (layer "F.Cu") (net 42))
 (segment (start 120.6755 61.0055) (end 120.6755 60.4975) (width 0.125) (layer "F.Cu") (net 42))
 (segment (start 121.158 62.016) (end 121.158 61.488) (width 0.125) (layer "F.Cu") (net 42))
 (segment (start 122.158 62.016) (end 122.158 60.740992) (width 0.125) (layer "F.Cu") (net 44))
 (segment (start 122.158 60.740992) (end 121.767504 60.350496) (width 0.125) (layer "F.Cu") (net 44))
 (segment (start 123.658 67.516) (end 125.4715 69.3295) (width 0.125) (layer "F.Cu") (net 47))
 (segment (start 125.4715 69.3295) (end 125.4715 71.1245) (width 0.125) (layer "F.Cu") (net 47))
 (segment (start 125.1465 69.5045) (end 125.1465 71.1655) (width 0.125) (layer "F.Cu") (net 57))
 (segment (start 123.658 68.016) (end 125.1465 69.5045) (width 0.125) (layer "F.Cu") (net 57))
 (segment (start 119.508 69.627619) (end 119.508 71.1655) (width 0.125) (layer "F.Cu") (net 60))
 (segment (start 119.158 68.516) (end 119.158 69.277619) (width 0.125) (layer "F.Cu") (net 60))
 (segment (start 119.158 69.277619) (end 119.508 69.627619) (width 0.125) (layer "F.Cu") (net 60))
 (segment (start 119.833 69.493) (end 119.833 71.1655) (width 0.125) (layer "F.Cu") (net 61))
 (segment (start 119.658 69.318) (end 119.833 69.493) (width 0.125) (layer "F.Cu") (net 61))
 (segment (start 119.658 68.516) (end 119.658 69.318) (width 0.125) (layer "F.Cu") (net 61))
 (segment (start 120.158 68.516) (end 120.158 71.1655) (width 0.125) (layer "F.Cu") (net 62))
 (segment (start 121.158 68.516) (end 121.158 68.779859) (width 0.125) (layer "F.Cu") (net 63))
 (segment (start 121.158 68.779859) (end 121.9155 69.537359) (width 0.125) (layer "F.Cu") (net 63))
 (segment (start 121.9155 69.537359) (end 121.9155 70.9115) (width 0.125) (layer "F.Cu") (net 63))
 (segment (start 122.2405 69.40274) (end 122.2405 70.9115) (width 0.125) (layer "F.Cu") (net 64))
 (segment (start 121.658 68.516) (end 121.658 68.82024) (width 0.125) (layer "F.Cu") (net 64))
 (segment (start 121.658 68.82024) (end 122.2405 69.40274) (width 0.125) (layer "F.Cu") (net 64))
 (segment (start 122.5655 69.26812) (end 122.5655 70.9115) (width 0.125) (layer "F.Cu") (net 65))
 (segment (start 122.158 68.86062) (end 122.5655 69.26812) (width 0.125) (layer "F.Cu") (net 65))
 (segment (start 122.158 68.516) (end 122.158 68.86062) (width 0.125) (layer "F.Cu") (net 65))
 (segment (start 122.658 68.516) (end 122.658 68.901) (width 0.125) (layer "F.Cu") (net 66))
 (segment (start 122.658 68.901) (end 122.8905 69.1335) (width 0.125) (layer "F.Cu") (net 66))
 (segment (start 122.8905 69.1335) (end 122.8905 70.9115) (width 0.125) (layer "F.Cu") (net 66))
 (segment (start 126.1925 66.5935) (end 127.8455 66.5935) (width 0.25) (layer "F.Cu") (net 82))
 (segment (start 123.658 64.516) (end 124.115 64.516) (width 0.25) (layer "F.Cu") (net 82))
 (segment (start 124.115 64.516) (end 126.1925 66.5935) (width 0.25) (layer "F.Cu") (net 82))
 (segment (start 114.0005 67.2135) (end 113.7465 67.2135) (width 0.125) (layer "F.Cu") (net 84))
 (segment (start 114.28764 67.2135) (end 114.0005 67.2135) (width 0.125) (layer "F.Cu") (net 84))
 (segment (start 116.48514 65.016) (end 114.28764 67.2135) (width 0.125) (layer "F.Cu") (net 84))
 (segment (start 117.158 65.016) (end 116.48514 65.016) (width 0.125) (layer "F.Cu") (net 84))
 (segment (start 123.658 65.016) (end 123.978604 65.016) (width 0.25) (layer "F.Cu") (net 85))
 (segment (start 126.064104 67.1015) (end 127.8455 67.1015) (width 0.25) (layer "F.Cu") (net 85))
 (segment (start 123.978604 65.016) (end 126.064104 67.1015) (width 0.25) (layer "F.Cu") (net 85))
 (segment (start 116.44476 65.516) (end 114.42226 67.5385) (width 0.125) (layer "F.Cu") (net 87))
 (segment (start 117.158 65.516) (end 116.44476 65.516) (width 0.125) (layer "F.Cu") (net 87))
 (segment (start 114.42226 67.5385) (end 114.0005 67.5385) (width 0.125) (layer "F.Cu") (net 87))
 (segment (start 123.842208 65.516) (end 125.429104 67.102896) (width 0.25) (layer "F.Cu") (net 88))
 (segment (start 125.429104 67.102896) (end 126.189708 67.8635) (width 0.25) (layer "F.Cu") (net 88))
 (segment (start 126.189708 67.8635) (end 126.1925 67.8635) (width 0.25) (layer "F.Cu") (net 88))
 (segment (start 123.658 65.516) (end 123.842208 65.516) (width 0.25) (layer "F.Cu") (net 88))
 (segment (start 117.158 66.016) (end 116.40438 66.016) (width 0.125) (layer "F.Cu") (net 91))
 (segment (start 116.40438 66.016) (end 114.55688 67.8635) (width 0.125) (layer "F.Cu") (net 91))
 (segment (start 114.55688 67.8635) (end 114.0005 67.8635) (width 0.125) (layer "F.Cu") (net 91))
 (segment (start 123.658 66.016) (end 126.4465 68.8045) (width 0.125) (layer "F.Cu") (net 92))
 (segment (start 126.4465 68.8045) (end 126.4465 71.1655) (width 0.125) (layer "F.Cu") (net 92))
 (segment (start 114.6915 68.1885) (end 114.0005 68.1885) (width 0.125) (layer "F.Cu") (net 95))
 (segment (start 116.364 66.516) (end 114.6915 68.1885) (width 0.125) (layer "F.Cu") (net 95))
 (segment (start 117.158 66.516) (end 116.364 66.516) (width 0.125) (layer "F.Cu") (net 95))
 (segment (start 123.658 66.516) (end 126.1215 68.9795) (width 0.125) (layer "F.Cu") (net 96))
 (segment (start 126.1215 68.9795) (end 126.1215 71.1655) (width 0.125) (layer "F.Cu") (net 96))
 (segment (start 123.658 67.016) (end 125.7965 69.1545) (width 0.125) (layer "F.Cu") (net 98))
 (segment (start 125.7965 69.1545) (end 125.7965 71.1655) (width 0.125) (layer "F.Cu") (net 98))
 (segment (start 118.7685 60.9475) (end 118.5725 60.7515) (width 0.25) (layer "F.Cu") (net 15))
 (segment (start 123.221603 64.716) (end 123.271603 64.766) (width 0.25) (layer "F.Cu") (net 15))
 (segment (start 122.99 64.716) (end 123.221603 64.716) (width 0.25) (layer "F.Cu") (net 15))
 (segment (start 121.908 63.766) (end 120.408 65.266) (width 0.25) (layer "F.Cu") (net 15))
 (segment (start 118.908 63.766) (end 120.408 65.266) (width 0.25) (layer "F.Cu") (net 15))
 (segment (start 118.908 62.516) (end 118.908 63.766) (width 0.25) (layer "F.Cu") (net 15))
 (segment (start 118.908 62.379604) (end 118.7685 62.240104) (width 0.25) (layer "F.Cu") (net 15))
 (segment (start 122.44 65.266) (end 122.99 64.716) (width 0.25) (layer "F.Cu") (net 15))
 (segment (start 123.238588 63.846588) (end 124.875412 63.846588) (width 0.125) (layer "F.Cu") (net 15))
 (segment (start 123.158 63.766) (end 123.238588 63.846588) (width 0.125) (layer "F.Cu") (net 15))
 (segment (start 118.7685 62.240104) (end 118.7685 60.9475) (width 0.25) (layer "F.Cu") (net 15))
 (segment (start 123.158 63.766) (end 121.908 63.766) (width 0.25) (layer "F.Cu") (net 15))
 (segment (start 118.908 62.516) (end 118.908 62.379604) (width 0.25) (layer "F.Cu") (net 15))
 (segment (start 124.875412 63.846588) (end 125.1765 63.5455) (width 0.125) (layer "F.Cu") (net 15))
 (segment (start 117.658 68.516) (end 117.658 70.556) (width 0.25) (layer "F.Cu") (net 24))
 (segment (start 117.158 63.016) (end 116.519 63.016) (width 0.25) (layer "F.Cu") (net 76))
 (segment (start 116.0325 62.5295) (end 114.5085 62.5295) (width 0.25) (layer "F.Cu") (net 76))
 (segment (start 116.519 63.016) (end 116.0325 62.5295) (width 0.25) (layer "F.Cu") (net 76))
 (segment (start 121.626 62.016) (end 121.6205 62.0215) (width 0.25) (layer "F.Cu") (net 43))
 (segment (start 121.6205 60.7515) (end 121.3665 60.4975) (width 0.25) (layer "F.Cu") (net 43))
 (segment (start 121.658 62.016) (end 121.626 62.016) (width 0.25) (layer "F.Cu") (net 43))
 (segment (start 121.6205 62.0215) (end 121.6205 60.7515) (width 0.25) (layer "F.Cu") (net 43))
 (segment (start 124.1605 61.5135) (end 124.1605 60.7515) (width 0.125) (layer "F.Cu") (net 46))
 (segment (start 123.158 62.016) (end 123.658 62.016) (width 0.125) (layer "F.Cu") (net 46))
 (segment (start 123.658 62.016) (end 124.1605 61.5135) (width 0.125) (layer "F.Cu") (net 46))
 (segment (start 117.0485 68.3715) (end 116.2865 69.1335) (width 0.25) (layer "F.Cu") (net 49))
 (segment (start 118.3455 68.0785) (end 117.3415 68.0785) (width 0.175) (layer "F.Cu") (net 49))
 (segment (start 116.2865 69.1335) (end 116.2865 70.6575) (width 0.25) (layer "F.Cu") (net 49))
 (segment (start 117.3415 68.0785) (end 117.0485 68.3715) (width 0.175) (layer "F.Cu") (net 49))
 (segment (start 118.408 68.016) (end 118.3455 68.0785) (width 0.175) (layer "F.Cu") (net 49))
 (segment (start 118.158 68.516) (end 118.158 69.302923) (width 0.175) (layer "F.Cu") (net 58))
 (segment (start 118.783 69.927923) (end 118.783 71.1655) (width 0.175) (layer "F.Cu") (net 58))
 (segment (start 118.158 69.302923) (end 118.783 69.927923) (width 0.175) (layer "F.Cu") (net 58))
 (segment (start 119.158 69.772593) (end 119.158 71.1655) (width 0.175) (layer "F.Cu") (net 59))
 (segment (start 118.658 68.516) (end 118.658 69.272593) (width 0.175) (layer "F.Cu") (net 59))
 (segment (start 118.658 69.272593) (end 119.158 69.772593) (width 0.175) (layer "F.Cu") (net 59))
 (segment (start 124.9225 62.2755) (end 125.9385 62.2755) (width 0.125) (layer "F.Cu") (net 68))
 (segment (start 123.658 63.516) (end 123.682 63.516) (width 0.125) (layer "F.Cu") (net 68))
 (segment (start 118.3185 62.0215) (end 117.0485 60.7515) (width 0.25) (layer "F.Cu") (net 68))
 (segment (start 118.408 62.516) (end 118.3185 62.4265) (width 0.25) (layer "F.Cu") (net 68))
 (segment (start 123.682 63.516) (end 124.9225 62.2755) (width 0.125) (layer "F.Cu") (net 68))
 (segment (start 118.3185 62.4265) (end 118.3185 62.0215) (width 0.25) (layer "F.Cu") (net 68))
 (segment (start 124.4855 61.6885) (end 124.4855 60.7515) (width 0.125) (layer "F.Cu") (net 75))
 (segment (start 123.658 62.516) (end 124.4855 61.6885) (width 0.125) (layer "F.Cu") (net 75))
 (segment (start 124.4855 60.7515) (end 124.4855 59.4105) (width 0.125) (layer "F.Cu") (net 75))
 (segment (start 124.4855 59.4105) (end 124.6685 59.2275) (width 0.125) (layer "F.Cu") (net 75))
 (segment (start 123.158 63.266) (end 123.5205 62.9035) (width 0.125) (layer "F.Cu") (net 78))
 (segment (start 123.5205 62.9035) (end 123.818508 62.9035) (width 0.125) (layer "F.Cu") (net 78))
 (segment (start 123.818508 62.9035) (end 125.1765 61.545508) (width 0.125) (layer "F.Cu") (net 78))
 (segment (start 125.1765 61.545508) (end 125.1765 61.5135) (width 0.125) (layer "F.Cu") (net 78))
 (segment (start 120.658 68.516) (end 120.658 70.096) (width 0.25) (layer "F.Cu") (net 45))
 (segment (start 123.158 68.516) (end 123.3985 68.7565) (width 0.25) (layer "F.Cu") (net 45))
 (segment (start 115.5245 61.0055) (end 114.5085 61.0055) (width 0.25) (layer "F.Cu") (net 45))
 (segment (start 115.6475 61.0055) (end 115.5245 61.0055) (width 0.25) (layer "F.Cu") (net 45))
 (segment (start 116.626 67.016) (end 115.0165 68.6255) (width 0.25) (layer "F.Cu") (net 45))
 (segment (start 117.158 67.016) (end 116.626 67.016) (width 0.25) (layer "F.Cu") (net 45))
 (segment (start 123.3985 68.7565) (end 123.3985 69.6415) (width 0.25) (layer "F.Cu") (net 45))
 (segment (start 117.158 62.516) (end 115.6475 61.0055) (width 0.25) (layer "F.Cu") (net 45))
 (segment (start 122.658 62.016) (end 122.658 60.519) (width 0.25) (layer "F.Cu") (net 45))
 (segment (start 114.15302 66.8885) (end 114.0005 66.8885) (width 0.125) (layer "F.Cu") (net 4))
 (segment (start 117.158 64.516) (end 116.52552 64.516) (width 0.125) (layer "F.Cu") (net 4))
 (segment (start 113.7875 66.8885) (end 113.7465 66.8885) (width 0.125) (layer "F.Cu") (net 4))
 (segment (start 116.52552 64.516) (end 114.22426 66.81726) (width 0.125) (layer "F.Cu") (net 4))
 (segment (start 114.0005 66.8885) (end 113.7875 66.8885) (width 0.125) (layer "F.Cu") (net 4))
 (segment (start 114.22426 66.81726) (end 114.15302 66.8885) (width 0.125) (layer "F.Cu") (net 4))
 (segment (start 116.5659 64.016) (end 114.0184 66.5635) (width 0.125) (layer "F.Cu") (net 1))
 (segment (start 117.158 64.016) (end 116.5659 64.016) (width 0.125) (layer "F.Cu") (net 1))
 (segment (start 114.0184 66.5635) (end 113.7765 66.5635) (width 0.125) (layer "F.Cu") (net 1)))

